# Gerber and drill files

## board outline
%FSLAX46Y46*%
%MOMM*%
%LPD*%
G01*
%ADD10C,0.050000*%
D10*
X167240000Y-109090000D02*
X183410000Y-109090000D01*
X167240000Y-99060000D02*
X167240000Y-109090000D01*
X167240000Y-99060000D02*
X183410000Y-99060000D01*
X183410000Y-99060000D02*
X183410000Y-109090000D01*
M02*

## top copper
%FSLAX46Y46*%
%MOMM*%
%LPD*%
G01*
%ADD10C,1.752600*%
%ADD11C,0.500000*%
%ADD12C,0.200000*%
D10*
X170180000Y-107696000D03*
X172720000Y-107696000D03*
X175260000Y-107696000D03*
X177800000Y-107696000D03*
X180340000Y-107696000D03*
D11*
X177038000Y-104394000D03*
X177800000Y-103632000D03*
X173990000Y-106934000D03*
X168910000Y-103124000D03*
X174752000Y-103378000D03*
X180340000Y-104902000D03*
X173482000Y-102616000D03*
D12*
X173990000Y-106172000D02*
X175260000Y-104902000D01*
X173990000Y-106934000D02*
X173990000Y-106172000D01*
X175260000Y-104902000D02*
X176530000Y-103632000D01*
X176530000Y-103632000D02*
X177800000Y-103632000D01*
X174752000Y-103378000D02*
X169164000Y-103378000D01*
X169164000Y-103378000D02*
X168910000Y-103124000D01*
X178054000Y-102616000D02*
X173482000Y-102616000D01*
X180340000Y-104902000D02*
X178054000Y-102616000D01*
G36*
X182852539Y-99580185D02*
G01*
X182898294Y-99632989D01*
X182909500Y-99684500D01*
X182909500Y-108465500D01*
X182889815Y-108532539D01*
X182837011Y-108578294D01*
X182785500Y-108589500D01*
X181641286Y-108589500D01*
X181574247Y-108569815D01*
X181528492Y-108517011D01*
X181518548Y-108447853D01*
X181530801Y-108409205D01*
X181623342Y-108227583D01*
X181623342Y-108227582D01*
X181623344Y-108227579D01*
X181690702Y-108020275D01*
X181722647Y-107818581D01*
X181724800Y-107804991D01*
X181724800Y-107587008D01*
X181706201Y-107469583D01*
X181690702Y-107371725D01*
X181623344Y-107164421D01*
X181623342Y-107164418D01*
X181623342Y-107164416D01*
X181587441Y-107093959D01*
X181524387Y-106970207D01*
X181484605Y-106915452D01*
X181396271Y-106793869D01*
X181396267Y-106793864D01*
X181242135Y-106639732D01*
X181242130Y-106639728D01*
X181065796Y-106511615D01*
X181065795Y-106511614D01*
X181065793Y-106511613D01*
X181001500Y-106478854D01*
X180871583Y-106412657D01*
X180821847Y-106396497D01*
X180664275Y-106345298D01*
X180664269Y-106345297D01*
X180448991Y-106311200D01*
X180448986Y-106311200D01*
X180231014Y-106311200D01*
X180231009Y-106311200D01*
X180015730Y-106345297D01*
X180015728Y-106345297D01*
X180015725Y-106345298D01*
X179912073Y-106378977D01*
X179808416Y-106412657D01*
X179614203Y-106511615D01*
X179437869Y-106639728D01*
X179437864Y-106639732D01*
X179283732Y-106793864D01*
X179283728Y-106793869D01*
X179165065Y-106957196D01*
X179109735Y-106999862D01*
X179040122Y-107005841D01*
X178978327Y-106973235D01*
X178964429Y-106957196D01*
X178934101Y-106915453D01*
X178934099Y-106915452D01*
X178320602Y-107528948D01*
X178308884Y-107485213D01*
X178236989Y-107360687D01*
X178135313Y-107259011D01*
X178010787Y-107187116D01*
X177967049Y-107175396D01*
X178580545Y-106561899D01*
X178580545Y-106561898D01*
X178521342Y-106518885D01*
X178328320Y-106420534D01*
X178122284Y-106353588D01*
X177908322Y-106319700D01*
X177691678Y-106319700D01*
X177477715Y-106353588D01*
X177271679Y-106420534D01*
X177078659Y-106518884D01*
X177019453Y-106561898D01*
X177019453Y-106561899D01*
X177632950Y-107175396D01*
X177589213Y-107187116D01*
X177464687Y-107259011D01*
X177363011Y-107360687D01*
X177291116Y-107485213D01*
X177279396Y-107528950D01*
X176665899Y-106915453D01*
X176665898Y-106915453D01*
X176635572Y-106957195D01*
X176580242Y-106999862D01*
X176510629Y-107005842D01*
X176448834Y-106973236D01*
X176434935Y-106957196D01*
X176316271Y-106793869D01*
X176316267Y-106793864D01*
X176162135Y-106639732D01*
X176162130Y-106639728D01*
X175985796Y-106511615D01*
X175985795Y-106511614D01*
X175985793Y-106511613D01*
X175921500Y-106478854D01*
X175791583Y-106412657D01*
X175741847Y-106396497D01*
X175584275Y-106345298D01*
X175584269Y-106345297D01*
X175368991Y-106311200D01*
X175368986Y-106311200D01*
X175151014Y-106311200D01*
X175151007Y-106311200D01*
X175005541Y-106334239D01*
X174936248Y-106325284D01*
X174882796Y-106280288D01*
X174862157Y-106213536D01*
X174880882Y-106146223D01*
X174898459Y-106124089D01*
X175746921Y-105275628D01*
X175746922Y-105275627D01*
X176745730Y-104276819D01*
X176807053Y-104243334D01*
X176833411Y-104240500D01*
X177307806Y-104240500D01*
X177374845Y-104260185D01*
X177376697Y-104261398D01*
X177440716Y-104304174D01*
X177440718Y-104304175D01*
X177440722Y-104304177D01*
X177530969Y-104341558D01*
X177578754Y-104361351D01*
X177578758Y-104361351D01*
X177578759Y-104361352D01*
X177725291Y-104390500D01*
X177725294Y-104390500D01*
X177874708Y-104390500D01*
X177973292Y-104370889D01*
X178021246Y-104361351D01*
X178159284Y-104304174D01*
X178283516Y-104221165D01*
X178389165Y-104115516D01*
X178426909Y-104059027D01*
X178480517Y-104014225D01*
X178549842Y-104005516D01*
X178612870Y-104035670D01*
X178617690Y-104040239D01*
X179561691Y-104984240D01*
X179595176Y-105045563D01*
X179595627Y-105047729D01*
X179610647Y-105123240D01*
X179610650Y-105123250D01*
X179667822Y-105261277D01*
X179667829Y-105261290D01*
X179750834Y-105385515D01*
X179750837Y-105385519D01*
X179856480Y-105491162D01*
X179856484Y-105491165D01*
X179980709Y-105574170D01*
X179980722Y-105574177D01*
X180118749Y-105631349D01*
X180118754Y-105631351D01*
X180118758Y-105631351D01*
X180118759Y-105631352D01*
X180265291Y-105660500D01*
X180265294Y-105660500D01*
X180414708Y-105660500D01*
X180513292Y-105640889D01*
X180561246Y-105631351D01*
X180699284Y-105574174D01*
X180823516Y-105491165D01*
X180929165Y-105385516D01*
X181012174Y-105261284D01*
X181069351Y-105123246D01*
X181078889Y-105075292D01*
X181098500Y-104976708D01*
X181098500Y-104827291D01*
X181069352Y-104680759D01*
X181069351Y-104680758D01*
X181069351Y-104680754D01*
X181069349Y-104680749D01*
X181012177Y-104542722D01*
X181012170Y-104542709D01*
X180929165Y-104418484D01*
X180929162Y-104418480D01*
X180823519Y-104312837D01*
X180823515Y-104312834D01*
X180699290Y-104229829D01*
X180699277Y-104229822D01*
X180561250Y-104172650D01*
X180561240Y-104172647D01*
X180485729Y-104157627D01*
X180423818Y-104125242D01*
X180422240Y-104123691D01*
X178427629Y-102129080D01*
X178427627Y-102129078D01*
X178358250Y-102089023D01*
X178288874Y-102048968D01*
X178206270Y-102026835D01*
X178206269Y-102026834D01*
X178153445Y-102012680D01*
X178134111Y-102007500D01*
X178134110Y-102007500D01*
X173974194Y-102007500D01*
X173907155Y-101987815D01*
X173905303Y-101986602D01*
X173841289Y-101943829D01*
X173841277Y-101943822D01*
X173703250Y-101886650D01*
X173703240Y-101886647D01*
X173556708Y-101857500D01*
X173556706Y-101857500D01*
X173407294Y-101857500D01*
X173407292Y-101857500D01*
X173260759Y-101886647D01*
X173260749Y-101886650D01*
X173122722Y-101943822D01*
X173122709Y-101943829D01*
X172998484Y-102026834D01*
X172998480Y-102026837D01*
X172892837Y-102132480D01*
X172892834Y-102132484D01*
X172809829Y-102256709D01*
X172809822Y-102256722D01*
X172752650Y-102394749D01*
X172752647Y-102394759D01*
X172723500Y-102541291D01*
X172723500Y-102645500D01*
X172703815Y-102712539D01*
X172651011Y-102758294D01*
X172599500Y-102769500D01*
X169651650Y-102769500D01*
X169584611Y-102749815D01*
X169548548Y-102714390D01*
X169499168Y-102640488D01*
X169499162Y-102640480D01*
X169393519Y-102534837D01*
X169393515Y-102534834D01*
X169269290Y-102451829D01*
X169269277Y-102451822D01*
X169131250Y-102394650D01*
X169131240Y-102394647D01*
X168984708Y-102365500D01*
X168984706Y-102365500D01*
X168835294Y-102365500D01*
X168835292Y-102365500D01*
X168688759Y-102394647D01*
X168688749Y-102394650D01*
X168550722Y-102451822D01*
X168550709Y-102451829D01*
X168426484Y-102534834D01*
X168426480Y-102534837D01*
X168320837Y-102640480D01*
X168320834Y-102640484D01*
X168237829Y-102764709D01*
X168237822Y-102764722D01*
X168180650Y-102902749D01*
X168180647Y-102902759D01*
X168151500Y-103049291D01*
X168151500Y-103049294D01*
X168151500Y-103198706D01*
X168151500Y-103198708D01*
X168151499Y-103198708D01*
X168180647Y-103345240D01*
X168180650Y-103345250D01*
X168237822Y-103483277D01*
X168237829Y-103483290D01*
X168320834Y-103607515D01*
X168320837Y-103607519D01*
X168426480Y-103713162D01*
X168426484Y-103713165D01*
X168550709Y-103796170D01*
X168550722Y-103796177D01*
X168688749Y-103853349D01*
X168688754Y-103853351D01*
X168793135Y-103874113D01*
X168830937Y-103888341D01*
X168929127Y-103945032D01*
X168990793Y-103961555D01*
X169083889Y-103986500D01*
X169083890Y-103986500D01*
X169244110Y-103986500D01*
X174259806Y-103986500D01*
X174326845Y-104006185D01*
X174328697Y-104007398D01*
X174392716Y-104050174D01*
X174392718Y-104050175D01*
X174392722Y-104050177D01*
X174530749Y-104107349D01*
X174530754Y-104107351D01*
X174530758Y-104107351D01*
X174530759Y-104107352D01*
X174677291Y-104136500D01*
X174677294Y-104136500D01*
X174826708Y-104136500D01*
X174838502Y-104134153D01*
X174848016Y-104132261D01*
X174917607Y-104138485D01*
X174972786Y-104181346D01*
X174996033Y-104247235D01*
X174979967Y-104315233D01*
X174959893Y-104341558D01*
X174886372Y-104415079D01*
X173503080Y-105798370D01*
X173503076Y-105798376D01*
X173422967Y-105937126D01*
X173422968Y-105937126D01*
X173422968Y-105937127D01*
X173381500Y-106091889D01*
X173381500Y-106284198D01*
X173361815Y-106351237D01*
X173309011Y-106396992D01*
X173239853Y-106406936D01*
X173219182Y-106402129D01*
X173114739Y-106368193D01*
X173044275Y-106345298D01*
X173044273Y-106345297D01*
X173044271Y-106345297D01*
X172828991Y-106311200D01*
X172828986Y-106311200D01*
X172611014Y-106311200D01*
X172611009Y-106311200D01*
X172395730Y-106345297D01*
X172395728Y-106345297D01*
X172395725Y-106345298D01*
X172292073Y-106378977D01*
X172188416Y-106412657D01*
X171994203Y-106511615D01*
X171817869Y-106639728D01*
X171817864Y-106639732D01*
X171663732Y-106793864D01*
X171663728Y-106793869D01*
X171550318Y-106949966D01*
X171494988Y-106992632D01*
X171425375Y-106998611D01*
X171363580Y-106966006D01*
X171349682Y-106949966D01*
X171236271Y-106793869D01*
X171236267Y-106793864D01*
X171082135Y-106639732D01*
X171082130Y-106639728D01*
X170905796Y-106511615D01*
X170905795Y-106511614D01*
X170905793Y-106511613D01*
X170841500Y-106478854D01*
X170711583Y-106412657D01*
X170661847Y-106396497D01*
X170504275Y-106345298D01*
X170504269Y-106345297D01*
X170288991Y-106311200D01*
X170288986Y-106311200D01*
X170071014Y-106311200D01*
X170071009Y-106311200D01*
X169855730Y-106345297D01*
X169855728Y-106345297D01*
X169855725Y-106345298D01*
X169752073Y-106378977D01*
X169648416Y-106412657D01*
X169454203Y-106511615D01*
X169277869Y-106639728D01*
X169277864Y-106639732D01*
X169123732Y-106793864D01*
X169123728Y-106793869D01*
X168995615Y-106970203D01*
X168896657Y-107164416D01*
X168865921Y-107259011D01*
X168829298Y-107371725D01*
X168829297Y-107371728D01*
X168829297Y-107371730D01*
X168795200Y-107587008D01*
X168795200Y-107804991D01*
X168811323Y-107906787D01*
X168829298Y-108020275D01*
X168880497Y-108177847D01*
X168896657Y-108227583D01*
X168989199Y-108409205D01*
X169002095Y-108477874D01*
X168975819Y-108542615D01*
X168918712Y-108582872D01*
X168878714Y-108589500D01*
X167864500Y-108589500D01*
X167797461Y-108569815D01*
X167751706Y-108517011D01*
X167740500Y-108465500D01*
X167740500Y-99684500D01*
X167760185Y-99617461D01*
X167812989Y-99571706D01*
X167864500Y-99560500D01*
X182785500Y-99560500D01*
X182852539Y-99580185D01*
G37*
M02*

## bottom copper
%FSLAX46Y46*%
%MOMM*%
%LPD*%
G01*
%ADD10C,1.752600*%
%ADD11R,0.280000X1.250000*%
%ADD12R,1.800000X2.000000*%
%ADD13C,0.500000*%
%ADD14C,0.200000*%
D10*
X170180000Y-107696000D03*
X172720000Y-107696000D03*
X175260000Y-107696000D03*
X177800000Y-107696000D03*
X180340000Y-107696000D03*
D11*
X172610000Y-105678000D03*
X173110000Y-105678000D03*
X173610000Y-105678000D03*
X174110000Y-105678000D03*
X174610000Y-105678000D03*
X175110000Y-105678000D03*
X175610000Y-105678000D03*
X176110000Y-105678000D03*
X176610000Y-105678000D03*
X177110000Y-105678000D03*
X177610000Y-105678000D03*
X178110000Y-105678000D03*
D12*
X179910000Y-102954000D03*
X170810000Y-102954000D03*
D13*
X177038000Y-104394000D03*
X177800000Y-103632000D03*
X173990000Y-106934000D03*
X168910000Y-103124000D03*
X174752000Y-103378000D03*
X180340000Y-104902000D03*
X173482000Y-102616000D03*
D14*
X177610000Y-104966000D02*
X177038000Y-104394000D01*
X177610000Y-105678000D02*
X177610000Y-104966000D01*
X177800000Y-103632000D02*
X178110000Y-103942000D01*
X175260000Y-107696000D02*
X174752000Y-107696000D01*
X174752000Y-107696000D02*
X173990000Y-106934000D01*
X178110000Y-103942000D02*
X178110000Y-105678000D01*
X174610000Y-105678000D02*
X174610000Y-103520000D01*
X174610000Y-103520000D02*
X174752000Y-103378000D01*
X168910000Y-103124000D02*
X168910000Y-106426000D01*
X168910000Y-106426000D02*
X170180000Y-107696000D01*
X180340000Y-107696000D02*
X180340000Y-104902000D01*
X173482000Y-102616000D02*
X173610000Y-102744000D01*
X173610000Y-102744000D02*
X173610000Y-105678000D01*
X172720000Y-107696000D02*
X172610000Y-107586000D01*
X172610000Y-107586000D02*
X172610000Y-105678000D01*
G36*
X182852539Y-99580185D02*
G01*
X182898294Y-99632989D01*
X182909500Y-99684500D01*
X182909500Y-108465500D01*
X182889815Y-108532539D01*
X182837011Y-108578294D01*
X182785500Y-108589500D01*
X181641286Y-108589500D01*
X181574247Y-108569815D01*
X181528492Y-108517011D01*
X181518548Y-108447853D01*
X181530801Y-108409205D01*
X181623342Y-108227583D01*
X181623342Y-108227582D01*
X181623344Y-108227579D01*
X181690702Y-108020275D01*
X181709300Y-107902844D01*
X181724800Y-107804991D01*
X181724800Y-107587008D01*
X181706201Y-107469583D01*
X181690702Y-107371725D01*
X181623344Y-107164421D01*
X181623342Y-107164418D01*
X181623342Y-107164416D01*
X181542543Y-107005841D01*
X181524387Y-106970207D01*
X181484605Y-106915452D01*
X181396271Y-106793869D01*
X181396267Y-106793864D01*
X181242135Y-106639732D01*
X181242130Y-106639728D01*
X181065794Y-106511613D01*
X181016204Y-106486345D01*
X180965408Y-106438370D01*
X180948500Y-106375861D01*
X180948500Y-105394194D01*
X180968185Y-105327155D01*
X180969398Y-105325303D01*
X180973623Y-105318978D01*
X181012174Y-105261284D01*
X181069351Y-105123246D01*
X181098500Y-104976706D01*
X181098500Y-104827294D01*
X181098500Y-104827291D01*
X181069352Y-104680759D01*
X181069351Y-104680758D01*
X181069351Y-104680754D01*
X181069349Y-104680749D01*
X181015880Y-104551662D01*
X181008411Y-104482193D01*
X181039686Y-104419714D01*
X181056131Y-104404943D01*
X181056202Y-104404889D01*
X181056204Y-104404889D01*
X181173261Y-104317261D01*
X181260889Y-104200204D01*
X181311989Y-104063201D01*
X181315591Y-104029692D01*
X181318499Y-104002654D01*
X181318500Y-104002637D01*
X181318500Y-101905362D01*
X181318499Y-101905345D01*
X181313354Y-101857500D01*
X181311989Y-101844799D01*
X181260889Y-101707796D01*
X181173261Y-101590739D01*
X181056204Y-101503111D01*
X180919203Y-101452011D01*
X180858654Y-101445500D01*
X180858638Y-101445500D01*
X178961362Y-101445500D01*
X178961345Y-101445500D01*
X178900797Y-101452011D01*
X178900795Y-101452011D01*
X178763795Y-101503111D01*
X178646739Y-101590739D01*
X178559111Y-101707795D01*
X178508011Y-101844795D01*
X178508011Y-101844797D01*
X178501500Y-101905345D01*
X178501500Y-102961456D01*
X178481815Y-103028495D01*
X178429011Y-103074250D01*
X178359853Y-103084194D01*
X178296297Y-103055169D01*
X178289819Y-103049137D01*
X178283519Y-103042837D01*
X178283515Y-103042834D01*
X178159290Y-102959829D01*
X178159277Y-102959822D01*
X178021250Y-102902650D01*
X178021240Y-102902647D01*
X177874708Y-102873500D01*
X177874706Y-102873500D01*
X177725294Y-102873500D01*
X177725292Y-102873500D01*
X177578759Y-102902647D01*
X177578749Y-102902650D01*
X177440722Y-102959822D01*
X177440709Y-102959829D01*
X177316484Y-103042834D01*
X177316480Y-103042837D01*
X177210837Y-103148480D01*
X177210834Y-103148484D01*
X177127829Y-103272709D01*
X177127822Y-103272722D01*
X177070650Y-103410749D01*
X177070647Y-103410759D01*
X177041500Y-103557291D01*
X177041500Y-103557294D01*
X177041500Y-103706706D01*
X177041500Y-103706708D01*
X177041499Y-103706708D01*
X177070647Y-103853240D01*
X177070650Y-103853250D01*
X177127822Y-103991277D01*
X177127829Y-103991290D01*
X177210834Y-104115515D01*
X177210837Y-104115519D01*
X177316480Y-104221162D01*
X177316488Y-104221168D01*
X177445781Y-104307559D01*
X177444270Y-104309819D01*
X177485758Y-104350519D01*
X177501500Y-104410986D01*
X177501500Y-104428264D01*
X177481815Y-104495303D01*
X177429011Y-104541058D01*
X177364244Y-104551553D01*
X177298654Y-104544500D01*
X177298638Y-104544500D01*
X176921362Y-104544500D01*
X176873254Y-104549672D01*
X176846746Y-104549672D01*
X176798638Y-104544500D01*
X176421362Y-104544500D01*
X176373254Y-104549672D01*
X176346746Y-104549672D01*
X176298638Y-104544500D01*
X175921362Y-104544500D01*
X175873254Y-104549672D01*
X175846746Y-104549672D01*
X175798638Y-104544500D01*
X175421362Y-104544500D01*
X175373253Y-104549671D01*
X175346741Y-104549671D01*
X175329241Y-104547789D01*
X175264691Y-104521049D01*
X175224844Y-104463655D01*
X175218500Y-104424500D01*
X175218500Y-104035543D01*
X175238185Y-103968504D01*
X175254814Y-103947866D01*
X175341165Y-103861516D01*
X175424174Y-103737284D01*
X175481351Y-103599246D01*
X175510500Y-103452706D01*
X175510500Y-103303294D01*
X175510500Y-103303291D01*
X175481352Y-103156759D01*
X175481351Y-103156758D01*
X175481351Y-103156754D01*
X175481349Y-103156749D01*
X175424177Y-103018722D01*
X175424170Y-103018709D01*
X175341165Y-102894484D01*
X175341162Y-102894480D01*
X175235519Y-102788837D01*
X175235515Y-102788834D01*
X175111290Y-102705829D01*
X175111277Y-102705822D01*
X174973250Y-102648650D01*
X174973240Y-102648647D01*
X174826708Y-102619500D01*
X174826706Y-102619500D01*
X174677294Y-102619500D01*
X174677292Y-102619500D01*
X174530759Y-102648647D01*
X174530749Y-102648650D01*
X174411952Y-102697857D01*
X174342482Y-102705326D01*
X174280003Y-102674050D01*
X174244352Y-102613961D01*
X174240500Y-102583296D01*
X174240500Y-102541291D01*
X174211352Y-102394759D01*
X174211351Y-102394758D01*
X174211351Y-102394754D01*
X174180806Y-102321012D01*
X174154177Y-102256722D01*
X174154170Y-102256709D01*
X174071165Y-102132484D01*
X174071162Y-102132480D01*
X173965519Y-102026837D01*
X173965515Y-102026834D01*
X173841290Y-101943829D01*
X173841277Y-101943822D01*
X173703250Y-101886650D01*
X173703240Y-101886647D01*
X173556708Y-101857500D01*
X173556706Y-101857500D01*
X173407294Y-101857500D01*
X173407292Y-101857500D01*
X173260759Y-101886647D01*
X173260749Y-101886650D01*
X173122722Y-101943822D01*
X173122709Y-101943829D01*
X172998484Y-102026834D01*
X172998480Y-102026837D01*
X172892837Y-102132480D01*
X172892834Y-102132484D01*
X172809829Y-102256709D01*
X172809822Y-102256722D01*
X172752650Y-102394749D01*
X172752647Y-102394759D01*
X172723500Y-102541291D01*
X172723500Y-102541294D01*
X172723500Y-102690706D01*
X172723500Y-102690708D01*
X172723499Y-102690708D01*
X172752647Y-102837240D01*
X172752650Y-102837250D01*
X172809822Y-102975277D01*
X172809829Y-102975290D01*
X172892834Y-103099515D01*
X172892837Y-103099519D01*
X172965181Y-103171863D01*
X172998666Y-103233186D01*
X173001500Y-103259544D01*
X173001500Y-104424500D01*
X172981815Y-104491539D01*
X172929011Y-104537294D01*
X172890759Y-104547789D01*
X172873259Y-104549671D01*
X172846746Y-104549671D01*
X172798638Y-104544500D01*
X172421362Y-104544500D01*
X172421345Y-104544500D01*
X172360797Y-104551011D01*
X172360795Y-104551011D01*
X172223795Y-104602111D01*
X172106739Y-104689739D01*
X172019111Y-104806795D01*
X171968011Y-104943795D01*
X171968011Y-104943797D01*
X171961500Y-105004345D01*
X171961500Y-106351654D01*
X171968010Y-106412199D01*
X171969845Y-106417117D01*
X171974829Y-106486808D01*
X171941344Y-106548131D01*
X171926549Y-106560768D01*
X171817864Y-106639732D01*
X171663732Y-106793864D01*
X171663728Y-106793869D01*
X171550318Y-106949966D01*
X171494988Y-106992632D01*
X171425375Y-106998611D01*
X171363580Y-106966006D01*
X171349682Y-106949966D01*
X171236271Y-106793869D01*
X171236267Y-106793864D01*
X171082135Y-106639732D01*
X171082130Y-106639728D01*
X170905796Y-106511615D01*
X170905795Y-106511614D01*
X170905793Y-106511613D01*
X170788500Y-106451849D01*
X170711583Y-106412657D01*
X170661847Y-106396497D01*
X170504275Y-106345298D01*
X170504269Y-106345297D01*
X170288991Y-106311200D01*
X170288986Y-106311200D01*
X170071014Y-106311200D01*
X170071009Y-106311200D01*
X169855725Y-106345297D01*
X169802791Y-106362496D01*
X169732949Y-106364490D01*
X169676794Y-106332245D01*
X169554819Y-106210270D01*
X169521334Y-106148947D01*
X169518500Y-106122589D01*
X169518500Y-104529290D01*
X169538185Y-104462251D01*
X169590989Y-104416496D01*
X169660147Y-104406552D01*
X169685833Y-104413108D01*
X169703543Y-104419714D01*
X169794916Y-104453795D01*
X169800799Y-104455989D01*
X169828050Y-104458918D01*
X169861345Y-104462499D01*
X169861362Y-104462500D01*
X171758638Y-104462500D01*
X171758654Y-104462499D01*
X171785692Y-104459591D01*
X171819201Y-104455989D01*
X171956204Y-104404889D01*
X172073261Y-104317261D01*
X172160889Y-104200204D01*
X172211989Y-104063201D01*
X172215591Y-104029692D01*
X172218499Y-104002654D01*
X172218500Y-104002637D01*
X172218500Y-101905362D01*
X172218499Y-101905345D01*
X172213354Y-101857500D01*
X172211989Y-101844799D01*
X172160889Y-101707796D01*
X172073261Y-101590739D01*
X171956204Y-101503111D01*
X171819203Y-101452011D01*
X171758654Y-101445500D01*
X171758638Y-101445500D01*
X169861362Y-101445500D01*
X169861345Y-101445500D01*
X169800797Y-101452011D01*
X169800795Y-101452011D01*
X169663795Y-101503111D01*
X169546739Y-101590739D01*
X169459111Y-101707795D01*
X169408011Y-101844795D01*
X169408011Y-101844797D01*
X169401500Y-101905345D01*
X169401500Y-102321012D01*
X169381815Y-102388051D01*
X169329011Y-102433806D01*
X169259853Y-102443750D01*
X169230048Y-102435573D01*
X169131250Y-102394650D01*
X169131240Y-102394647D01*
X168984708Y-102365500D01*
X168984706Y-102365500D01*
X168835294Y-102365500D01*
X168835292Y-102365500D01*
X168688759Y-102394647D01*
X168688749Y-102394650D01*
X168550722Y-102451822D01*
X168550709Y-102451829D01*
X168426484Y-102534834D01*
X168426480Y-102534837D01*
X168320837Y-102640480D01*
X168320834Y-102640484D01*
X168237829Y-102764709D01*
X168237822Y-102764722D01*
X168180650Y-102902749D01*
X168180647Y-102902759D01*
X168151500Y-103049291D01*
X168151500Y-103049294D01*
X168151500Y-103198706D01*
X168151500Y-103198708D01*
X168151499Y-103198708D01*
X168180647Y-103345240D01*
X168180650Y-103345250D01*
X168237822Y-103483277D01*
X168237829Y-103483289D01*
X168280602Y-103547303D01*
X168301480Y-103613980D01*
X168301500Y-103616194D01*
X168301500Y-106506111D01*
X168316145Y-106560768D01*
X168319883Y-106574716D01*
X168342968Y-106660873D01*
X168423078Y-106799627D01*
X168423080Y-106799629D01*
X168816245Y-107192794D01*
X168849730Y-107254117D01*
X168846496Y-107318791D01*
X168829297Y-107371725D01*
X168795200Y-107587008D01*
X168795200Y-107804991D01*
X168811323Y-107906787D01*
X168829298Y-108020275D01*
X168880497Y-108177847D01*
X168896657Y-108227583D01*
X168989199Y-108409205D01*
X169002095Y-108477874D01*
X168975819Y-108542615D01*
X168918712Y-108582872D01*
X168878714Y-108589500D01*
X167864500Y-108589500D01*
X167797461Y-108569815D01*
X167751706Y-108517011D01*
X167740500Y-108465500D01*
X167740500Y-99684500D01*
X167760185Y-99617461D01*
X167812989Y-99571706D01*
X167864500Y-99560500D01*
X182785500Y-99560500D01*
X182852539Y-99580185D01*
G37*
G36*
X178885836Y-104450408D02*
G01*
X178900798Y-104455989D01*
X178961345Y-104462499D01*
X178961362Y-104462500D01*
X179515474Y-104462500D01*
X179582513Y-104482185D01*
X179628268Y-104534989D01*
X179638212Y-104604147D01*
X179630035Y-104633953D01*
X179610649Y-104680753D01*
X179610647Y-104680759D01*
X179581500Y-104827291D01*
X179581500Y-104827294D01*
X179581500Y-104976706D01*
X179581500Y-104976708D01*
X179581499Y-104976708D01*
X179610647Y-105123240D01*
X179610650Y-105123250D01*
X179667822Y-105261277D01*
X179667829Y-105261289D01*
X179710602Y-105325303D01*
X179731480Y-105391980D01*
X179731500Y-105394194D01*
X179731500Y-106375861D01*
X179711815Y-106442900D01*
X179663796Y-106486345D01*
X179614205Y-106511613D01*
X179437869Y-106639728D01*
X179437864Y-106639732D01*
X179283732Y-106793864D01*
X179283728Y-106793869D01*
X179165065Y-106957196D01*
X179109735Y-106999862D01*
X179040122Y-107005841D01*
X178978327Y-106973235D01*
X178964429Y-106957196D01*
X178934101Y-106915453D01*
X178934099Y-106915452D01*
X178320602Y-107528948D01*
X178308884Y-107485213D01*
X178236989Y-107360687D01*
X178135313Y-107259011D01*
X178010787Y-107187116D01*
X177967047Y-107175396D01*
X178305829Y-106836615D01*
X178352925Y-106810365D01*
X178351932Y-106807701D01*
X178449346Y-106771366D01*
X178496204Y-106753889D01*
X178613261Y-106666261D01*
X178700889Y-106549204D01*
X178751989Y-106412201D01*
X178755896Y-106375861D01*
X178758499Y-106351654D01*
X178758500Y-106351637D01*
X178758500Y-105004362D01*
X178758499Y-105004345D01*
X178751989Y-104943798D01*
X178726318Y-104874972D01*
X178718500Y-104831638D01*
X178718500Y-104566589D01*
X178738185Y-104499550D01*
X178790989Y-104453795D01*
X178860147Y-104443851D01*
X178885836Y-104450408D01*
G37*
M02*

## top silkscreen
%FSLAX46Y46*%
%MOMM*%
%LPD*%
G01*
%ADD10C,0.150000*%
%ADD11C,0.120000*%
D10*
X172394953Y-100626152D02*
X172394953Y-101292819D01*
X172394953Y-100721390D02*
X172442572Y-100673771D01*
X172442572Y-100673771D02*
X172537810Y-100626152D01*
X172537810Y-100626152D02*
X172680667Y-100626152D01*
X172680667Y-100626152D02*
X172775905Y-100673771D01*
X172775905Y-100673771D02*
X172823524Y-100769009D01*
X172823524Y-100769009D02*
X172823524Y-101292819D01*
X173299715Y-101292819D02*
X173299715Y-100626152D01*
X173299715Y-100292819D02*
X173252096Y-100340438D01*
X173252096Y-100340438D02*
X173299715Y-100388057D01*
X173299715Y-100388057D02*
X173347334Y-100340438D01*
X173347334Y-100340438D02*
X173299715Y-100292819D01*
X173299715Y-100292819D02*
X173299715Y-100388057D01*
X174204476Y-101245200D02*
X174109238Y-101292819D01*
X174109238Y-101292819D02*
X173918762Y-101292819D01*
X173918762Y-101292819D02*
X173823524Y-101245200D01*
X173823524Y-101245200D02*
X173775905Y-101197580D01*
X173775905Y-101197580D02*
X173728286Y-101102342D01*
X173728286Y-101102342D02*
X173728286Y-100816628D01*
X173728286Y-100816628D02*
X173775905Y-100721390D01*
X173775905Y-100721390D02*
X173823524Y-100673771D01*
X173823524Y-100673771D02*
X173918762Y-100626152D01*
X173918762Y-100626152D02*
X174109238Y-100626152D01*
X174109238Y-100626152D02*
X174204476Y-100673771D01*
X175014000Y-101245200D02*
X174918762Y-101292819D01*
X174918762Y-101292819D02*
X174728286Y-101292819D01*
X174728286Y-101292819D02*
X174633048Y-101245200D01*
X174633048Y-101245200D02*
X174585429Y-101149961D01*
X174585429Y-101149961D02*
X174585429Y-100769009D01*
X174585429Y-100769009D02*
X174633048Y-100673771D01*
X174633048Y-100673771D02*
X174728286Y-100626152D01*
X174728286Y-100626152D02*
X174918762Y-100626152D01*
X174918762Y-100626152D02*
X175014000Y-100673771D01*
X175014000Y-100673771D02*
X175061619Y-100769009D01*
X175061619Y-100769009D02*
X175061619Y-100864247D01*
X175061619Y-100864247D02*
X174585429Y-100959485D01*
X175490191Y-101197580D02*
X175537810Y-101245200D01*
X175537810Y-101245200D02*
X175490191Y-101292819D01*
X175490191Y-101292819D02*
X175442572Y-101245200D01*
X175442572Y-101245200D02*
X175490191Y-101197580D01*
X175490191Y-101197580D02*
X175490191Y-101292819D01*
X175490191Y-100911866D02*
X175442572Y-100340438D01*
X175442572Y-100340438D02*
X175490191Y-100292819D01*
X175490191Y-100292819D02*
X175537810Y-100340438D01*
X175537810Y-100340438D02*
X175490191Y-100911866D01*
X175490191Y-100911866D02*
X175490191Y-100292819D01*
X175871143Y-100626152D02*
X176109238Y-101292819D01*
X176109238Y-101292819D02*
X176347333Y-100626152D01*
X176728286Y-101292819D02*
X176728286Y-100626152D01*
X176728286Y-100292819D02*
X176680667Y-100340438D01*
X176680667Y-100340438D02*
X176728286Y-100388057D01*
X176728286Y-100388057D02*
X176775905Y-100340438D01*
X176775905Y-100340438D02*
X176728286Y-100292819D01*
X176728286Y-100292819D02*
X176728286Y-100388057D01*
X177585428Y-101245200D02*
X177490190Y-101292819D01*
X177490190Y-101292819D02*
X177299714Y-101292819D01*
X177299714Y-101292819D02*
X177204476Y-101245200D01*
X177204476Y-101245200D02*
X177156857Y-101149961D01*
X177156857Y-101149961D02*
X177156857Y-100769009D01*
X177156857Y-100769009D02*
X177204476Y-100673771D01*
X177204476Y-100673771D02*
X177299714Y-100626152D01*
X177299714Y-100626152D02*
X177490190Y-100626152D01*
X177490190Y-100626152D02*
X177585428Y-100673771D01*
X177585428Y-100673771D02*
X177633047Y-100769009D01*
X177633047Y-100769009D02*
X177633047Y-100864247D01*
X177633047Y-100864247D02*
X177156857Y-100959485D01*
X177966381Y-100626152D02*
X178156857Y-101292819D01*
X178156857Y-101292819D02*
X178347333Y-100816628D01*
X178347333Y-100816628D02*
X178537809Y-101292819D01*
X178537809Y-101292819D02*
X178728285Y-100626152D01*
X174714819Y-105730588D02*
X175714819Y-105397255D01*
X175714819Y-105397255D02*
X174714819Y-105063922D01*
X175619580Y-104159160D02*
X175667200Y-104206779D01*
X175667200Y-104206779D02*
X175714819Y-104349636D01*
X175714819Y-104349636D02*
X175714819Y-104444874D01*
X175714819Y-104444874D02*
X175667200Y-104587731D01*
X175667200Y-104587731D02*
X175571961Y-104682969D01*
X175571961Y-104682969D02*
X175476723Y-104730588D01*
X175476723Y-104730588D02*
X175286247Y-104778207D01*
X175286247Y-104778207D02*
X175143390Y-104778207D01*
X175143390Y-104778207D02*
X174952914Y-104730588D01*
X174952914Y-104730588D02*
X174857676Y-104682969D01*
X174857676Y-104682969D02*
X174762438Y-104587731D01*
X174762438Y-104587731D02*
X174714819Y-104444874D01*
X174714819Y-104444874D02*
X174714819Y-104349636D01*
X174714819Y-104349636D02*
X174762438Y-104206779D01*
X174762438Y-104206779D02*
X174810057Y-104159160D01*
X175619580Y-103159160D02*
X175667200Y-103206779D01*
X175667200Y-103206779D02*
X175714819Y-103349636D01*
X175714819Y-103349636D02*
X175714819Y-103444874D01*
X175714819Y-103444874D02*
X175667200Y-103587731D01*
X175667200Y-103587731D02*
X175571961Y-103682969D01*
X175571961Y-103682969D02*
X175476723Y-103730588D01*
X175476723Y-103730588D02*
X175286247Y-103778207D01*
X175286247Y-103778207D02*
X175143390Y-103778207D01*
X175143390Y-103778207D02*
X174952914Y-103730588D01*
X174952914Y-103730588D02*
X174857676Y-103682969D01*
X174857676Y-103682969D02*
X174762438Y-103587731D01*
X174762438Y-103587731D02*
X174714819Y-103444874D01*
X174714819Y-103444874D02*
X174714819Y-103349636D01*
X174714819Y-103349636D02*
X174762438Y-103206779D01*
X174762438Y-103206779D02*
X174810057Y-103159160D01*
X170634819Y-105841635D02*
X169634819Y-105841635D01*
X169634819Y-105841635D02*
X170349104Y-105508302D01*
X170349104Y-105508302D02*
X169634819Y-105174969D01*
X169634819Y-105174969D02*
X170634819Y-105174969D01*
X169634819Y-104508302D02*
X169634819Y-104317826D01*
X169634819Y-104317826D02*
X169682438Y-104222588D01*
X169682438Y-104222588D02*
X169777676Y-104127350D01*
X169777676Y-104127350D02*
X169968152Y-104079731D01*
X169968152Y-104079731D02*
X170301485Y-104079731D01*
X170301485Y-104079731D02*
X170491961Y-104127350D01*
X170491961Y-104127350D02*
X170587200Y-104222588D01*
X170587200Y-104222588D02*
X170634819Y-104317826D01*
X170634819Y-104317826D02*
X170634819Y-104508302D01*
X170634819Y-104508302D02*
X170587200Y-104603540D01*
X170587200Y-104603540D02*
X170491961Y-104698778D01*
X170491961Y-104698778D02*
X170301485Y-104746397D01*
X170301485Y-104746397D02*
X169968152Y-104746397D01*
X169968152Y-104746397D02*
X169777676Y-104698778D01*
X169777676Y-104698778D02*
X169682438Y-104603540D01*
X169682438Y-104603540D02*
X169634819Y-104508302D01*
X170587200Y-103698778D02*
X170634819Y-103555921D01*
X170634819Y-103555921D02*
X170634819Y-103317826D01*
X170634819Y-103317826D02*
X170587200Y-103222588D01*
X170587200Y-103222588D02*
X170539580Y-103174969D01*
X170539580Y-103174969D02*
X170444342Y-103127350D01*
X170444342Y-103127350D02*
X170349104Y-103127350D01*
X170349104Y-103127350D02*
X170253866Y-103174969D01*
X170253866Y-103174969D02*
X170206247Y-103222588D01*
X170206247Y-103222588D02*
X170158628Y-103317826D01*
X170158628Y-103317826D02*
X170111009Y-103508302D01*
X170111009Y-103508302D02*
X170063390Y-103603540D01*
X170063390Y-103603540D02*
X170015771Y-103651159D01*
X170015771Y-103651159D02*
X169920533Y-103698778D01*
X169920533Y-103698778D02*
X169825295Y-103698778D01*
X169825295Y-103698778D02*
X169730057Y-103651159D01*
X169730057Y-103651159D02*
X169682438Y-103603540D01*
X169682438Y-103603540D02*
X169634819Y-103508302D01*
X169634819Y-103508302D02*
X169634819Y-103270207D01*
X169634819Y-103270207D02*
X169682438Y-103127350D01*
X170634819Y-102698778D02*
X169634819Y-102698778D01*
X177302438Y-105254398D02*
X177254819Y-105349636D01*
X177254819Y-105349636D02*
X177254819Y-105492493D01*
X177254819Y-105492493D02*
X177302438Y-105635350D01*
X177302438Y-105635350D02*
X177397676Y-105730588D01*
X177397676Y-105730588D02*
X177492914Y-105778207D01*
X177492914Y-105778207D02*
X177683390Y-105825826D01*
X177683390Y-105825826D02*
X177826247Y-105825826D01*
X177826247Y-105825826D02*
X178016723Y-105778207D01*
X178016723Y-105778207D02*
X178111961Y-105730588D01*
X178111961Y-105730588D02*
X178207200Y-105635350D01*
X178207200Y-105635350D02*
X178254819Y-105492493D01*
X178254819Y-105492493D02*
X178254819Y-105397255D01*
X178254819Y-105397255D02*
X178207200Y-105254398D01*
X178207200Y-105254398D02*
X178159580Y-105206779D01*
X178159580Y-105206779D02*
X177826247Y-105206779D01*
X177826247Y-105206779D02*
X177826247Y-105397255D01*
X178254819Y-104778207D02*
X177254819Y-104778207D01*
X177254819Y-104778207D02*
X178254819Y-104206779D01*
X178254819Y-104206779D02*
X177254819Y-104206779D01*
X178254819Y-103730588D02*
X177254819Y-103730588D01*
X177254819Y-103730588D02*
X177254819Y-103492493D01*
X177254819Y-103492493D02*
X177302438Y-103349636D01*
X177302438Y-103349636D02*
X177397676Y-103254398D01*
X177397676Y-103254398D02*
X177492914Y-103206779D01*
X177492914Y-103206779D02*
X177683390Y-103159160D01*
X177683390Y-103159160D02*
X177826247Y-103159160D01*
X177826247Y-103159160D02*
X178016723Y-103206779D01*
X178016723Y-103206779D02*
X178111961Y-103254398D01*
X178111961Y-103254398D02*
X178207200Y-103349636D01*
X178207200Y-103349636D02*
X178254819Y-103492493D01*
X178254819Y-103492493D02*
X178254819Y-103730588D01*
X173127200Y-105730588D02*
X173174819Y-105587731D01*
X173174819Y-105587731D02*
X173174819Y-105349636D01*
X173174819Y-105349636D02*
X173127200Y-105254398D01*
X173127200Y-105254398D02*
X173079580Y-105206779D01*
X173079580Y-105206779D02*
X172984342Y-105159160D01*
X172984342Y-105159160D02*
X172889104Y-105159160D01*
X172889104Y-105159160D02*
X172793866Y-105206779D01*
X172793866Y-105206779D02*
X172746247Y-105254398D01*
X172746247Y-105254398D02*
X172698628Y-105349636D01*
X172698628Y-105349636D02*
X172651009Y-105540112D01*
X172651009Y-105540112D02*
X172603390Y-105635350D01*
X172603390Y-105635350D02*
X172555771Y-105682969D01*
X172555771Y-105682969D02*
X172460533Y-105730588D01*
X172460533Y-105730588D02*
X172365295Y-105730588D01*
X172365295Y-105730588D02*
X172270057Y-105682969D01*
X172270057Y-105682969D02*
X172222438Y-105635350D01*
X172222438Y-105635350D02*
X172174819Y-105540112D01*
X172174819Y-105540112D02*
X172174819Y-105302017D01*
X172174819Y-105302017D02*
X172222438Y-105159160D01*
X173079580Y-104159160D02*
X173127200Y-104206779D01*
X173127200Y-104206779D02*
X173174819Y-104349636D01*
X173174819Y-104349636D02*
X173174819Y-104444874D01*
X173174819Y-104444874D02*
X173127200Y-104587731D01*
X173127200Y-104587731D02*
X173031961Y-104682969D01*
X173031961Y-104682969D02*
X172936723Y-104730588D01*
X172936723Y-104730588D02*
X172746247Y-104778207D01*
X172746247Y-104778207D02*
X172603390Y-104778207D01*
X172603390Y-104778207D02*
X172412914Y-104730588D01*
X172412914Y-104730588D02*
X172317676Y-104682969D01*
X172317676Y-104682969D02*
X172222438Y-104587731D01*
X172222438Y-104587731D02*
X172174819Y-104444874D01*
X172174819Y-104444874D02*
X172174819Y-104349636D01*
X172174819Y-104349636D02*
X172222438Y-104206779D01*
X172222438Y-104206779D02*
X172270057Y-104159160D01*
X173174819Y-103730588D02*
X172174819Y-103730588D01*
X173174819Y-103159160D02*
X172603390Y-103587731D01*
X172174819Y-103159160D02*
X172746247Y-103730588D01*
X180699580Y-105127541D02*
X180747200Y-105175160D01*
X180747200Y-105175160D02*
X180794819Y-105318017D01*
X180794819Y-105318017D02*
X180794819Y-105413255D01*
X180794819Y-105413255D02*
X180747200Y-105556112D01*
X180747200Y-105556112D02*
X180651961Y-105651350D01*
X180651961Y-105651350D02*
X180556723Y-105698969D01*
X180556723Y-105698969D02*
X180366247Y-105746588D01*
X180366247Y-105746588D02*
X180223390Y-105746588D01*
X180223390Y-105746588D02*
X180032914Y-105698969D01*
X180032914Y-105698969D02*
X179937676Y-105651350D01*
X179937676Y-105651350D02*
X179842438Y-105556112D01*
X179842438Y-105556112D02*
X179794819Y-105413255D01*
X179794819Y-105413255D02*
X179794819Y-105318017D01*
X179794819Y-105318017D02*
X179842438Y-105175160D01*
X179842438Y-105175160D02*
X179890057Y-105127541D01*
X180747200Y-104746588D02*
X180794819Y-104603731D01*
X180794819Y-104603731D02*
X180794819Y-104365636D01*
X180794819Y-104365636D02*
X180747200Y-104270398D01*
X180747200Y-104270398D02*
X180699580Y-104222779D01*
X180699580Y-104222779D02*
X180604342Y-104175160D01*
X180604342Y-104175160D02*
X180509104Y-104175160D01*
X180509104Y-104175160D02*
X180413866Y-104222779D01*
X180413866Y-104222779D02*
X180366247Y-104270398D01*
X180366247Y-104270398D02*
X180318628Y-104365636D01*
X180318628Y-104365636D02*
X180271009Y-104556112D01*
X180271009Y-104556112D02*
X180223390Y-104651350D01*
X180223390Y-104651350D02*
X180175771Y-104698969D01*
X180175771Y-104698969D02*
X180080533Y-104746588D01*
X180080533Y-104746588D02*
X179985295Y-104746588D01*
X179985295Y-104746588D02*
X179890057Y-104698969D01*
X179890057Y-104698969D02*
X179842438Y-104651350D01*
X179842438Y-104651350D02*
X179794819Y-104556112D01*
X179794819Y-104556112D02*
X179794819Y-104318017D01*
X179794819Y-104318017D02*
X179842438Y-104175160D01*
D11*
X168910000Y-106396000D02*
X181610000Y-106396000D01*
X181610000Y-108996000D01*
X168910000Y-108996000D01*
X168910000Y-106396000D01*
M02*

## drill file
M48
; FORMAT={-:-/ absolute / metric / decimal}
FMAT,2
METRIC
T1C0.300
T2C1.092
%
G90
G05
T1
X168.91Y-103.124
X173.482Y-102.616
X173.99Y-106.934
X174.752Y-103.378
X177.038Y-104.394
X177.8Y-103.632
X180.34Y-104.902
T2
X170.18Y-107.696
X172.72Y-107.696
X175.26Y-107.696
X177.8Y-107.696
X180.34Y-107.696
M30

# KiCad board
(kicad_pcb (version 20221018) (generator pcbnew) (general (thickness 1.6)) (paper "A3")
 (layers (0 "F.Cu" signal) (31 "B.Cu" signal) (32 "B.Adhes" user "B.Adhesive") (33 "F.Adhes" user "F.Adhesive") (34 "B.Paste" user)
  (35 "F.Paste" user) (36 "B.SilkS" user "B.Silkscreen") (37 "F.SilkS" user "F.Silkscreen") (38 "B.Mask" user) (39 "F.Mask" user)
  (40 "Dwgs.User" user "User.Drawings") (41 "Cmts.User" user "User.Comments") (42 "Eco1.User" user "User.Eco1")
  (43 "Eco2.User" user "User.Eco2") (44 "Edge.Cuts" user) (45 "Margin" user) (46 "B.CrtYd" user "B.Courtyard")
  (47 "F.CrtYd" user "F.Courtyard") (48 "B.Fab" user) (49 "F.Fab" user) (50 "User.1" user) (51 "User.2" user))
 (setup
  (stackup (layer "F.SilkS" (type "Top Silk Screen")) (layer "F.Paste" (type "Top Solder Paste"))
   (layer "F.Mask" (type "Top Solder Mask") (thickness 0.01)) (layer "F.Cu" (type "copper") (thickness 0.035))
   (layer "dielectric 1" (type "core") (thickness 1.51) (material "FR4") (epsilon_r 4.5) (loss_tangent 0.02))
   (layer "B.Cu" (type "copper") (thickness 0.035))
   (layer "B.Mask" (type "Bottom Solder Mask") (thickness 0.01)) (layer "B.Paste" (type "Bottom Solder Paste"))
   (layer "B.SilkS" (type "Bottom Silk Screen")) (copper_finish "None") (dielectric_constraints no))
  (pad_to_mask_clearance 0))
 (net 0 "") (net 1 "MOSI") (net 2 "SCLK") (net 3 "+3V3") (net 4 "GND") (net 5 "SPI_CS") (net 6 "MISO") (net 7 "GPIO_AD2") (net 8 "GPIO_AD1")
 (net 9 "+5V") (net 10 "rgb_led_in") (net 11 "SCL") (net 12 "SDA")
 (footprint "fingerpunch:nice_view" (layer "F.Cu") (at 175.26 91.216)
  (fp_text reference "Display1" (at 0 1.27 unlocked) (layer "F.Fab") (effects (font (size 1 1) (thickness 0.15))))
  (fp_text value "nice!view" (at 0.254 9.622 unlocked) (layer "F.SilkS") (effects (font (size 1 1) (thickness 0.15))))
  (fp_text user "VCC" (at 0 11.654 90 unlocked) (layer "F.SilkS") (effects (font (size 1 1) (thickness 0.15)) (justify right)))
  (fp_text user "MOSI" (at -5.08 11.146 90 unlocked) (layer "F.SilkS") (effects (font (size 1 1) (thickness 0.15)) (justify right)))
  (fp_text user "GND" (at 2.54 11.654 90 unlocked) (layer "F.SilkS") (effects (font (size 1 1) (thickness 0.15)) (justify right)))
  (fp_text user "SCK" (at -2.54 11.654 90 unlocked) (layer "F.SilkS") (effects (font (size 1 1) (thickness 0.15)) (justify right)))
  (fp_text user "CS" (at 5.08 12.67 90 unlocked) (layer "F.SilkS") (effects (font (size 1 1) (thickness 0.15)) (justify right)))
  (fp_rect (start -6.35 15.18) (end 6.35 17.78) (stroke (width 0.12) (type solid)) (fill none) (layer "F.SilkS"))
  (pad "1" thru_hole circle (at -5.08 16.48) (size 1.7526 1.7526) (drill 1.0922) (layers "*.Cu" "*.Mask") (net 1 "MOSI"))
  (pad "2" thru_hole circle (at -2.54 16.48) (size 1.7526 1.7526) (drill 1.0922) (layers "*.Cu" "*.Mask") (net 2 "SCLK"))
  (pad "3" thru_hole circle (at 0 16.48) (size 1.7526 1.7526) (drill 1.0922) (layers "*.Cu" "*.Mask") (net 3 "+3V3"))
  (pad "4" thru_hole circle (at 2.54 16.48) (size 1.7526 1.7526) (drill 1.0922) (layers "*.Cu" "*.Mask") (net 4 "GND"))
  (pad "5" thru_hole circle (at 5.08 16.48) (size 1.7526 1.7526) (drill 1.0922) (layers "*.Cu" "*.Mask") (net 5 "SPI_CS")))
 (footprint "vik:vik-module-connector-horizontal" (layer "B.Cu") (at 175.36 103.64)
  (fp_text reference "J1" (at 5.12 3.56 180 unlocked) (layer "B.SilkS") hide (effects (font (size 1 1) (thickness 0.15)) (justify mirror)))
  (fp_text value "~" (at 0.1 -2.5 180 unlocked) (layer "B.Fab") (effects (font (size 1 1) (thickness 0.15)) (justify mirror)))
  (pad "1" smd rect (at -2.75 2.038) (size 0.28 1.25) (layers "B.Cu" "B.Paste" "B.Mask") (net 2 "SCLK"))
  (pad "2" smd rect (at -2.25 2.038) (size 0.28 1.25) (layers "B.Cu" "B.Paste" "B.Mask") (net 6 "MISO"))
  (pad "3" smd rect (at -1.75 2.038) (size 0.28 1.25) (layers "B.Cu" "B.Paste" "B.Mask") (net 5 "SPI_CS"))
  (pad "4" smd rect (at -1.25 2.038) (size 0.28 1.25) (layers "B.Cu" "B.Paste" "B.Mask") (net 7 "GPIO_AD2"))
  (pad "5" smd rect (at -0.75 2.038) (size 0.28 1.25) (layers "B.Cu" "B.Paste" "B.Mask") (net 1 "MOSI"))
  (pad "6" smd rect (at -0.25 2.038) (size 0.28 1.25) (layers "B.Cu" "B.Paste" "B.Mask") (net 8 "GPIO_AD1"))
  (pad "7" smd rect (at 0.25 2.038) (size 0.28 1.25) (layers "B.Cu" "B.Paste" "B.Mask") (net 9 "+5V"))
  (pad "8" smd rect (at 0.75 2.038) (size 0.28 1.25) (layers "B.Cu" "B.Paste" "B.Mask") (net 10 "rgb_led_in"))
  (pad "9" smd rect (at 1.25 2.038) (size 0.28 1.25) (layers "B.Cu" "B.Paste" "B.Mask") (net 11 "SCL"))
  (pad "10" smd rect (at 1.75 2.038) (size 0.28 1.25) (layers "B.Cu" "B.Paste" "B.Mask") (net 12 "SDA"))
  (pad "11" smd rect (at 2.25 2.038) (size 0.28 1.25) (layers "B.Cu" "B.Paste" "B.Mask") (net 4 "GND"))
  (pad "12" smd rect (at 2.75 2.038) (size 0.28 1.25) (layers "B.Cu" "B.Paste" "B.Mask") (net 3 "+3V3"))
  (pad "13" smd rect (at 4.55 -0.686) (size 1.8 2) (layers "B.Cu" "B.Paste" "B.Mask"))
  (pad "14" smd rect (at -4.55 -0.686) (size 1.8 2) (layers "B.Cu" "B.Paste" "B.Mask")))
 (gr_line (start 167.24 109.09) (end 183.41 109.09) (stroke (width 0.05) (type default)) (layer "Edge.Cuts"))
 (gr_line (start 167.24 99.06) (end 167.24 109.09) (stroke (width 0.05) (type default)) (layer "Edge.Cuts"))
 (gr_line (start 167.24 99.06) (end 183.41 99.06) (stroke (width 0.05) (type default)) (layer "Edge.Cuts"))
 (gr_line (start 183.41 99.06) (end 183.41 109.09) (stroke (width 0.05) (type default)) (layer "Edge.Cuts"))
 (via (at 177.038 104.394) (size 0.5) (drill 0.3) (layers "F.Cu" "B.Cu") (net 4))
 (segment (start 177.61 104.966) (end 177.038 104.394) (width 0.2) (layer "B.Cu") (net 4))
 (segment (start 177.61 105.678) (end 177.61 104.966) (width 0.2) (layer "B.Cu") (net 4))
 (segment (start 173.99 106.172) (end 175.26 104.902) (width 0.2) (layer "F.Cu") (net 3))
 (segment (start 173.99 106.934) (end 173.99 106.172) (width 0.2) (layer "F.Cu") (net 3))
 (segment (start 175.26 104.902) (end 176.53 103.632) (width 0.2) (layer "F.Cu") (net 3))
 (segment (start 176.53 103.632) (end 177.8 103.632) (width 0.2) (layer "F.Cu") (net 3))
 (via (at 177.8 103.632) (size 0.5) (drill 0.3) (layers "F.Cu" "B.Cu") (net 3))
 (via (at 173.99 106.934) (size 0.5) (drill 0.3) (layers "F.Cu" "B.Cu") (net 3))
 (segment (start 177.8 103.632) (end 178.11 103.942) (width 0.2) (layer "B.Cu") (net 3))
 (segment (start 175.26 107.696) (end 174.752 107.696) (width 0.2) (layer "B.Cu") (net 3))
 (segment (start 174.752 107.696) (end 173.99 106.934) (width 0.2) (layer "B.Cu") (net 3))
 (segment (start 178.11 103.942) (end 178.11 105.678) (width 0.2) (layer "B.Cu") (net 3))
 (segment (start 174.752 103.378) (end 169.164 103.378) (width 0.2) (layer "F.Cu") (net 1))
 (segment (start 169.164 103.378) (end 168.91 103.124) (width 0.2) (layer "F.Cu") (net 1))
 (via (at 168.91 103.124) (size 0.5) (drill 0.3) (layers "F.Cu" "B.Cu") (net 1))
 (via (at 174.752 103.378) (size 0.5) (drill 0.3) (layers "F.Cu" "B.Cu") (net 1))
 (segment (start 174.61 105.678) (end 174.61 103.52) (width 0.2) (layer "B.Cu") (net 1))
 (segment (start 174.61 103.52) (end 174.752 103.378) (width 0.2) (layer "B.Cu") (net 1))
 (segment (start 168.91 103.124) (end 168.91 106.426) (width 0.2) (layer "B.Cu") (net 1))
 (segment (start 168.91 106.426) (end 170.18 107.696) (width 0.2) (layer "B.Cu") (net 1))
 (segment (start 178.054 102.616) (end 173.482 102.616) (width 0.2) (layer "F.Cu") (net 5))
 (segment (start 180.34 104.902) (end 178.054 102.616) (width 0.2) (layer "F.Cu") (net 5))
 (via (at 180.34 104.902) (size 0.5) (drill 0.3) (layers "F.Cu" "B.Cu") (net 5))
 (via (at 173.482 102.616) (size 0.5) (drill 0.3) (layers "F.Cu" "B.Cu") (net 5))
 (segment (start 180.34 107.696) (end 180.34 104.902) (width 0.2) (layer "B.Cu") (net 5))
 (segment (start 173.482 102.616) (end 173.61 102.744) (width 0.2) (layer "B.Cu") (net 5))
 (segment (start 173.61 102.744) (end 173.61 105.678) (width 0.2) (layer "B.Cu") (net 5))
 (segment (start 172.72 107.696) (end 172.61 107.586) (width 0.2) (layer "B.Cu") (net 2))
 (segment (start 172.61 107.586) (end 172.61 105.678) (width 0.2) (layer "B.Cu") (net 2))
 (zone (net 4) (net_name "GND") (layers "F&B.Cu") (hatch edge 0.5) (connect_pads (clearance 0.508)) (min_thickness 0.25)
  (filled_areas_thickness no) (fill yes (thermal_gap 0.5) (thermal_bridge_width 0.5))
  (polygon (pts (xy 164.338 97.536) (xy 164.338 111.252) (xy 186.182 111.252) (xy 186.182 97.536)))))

